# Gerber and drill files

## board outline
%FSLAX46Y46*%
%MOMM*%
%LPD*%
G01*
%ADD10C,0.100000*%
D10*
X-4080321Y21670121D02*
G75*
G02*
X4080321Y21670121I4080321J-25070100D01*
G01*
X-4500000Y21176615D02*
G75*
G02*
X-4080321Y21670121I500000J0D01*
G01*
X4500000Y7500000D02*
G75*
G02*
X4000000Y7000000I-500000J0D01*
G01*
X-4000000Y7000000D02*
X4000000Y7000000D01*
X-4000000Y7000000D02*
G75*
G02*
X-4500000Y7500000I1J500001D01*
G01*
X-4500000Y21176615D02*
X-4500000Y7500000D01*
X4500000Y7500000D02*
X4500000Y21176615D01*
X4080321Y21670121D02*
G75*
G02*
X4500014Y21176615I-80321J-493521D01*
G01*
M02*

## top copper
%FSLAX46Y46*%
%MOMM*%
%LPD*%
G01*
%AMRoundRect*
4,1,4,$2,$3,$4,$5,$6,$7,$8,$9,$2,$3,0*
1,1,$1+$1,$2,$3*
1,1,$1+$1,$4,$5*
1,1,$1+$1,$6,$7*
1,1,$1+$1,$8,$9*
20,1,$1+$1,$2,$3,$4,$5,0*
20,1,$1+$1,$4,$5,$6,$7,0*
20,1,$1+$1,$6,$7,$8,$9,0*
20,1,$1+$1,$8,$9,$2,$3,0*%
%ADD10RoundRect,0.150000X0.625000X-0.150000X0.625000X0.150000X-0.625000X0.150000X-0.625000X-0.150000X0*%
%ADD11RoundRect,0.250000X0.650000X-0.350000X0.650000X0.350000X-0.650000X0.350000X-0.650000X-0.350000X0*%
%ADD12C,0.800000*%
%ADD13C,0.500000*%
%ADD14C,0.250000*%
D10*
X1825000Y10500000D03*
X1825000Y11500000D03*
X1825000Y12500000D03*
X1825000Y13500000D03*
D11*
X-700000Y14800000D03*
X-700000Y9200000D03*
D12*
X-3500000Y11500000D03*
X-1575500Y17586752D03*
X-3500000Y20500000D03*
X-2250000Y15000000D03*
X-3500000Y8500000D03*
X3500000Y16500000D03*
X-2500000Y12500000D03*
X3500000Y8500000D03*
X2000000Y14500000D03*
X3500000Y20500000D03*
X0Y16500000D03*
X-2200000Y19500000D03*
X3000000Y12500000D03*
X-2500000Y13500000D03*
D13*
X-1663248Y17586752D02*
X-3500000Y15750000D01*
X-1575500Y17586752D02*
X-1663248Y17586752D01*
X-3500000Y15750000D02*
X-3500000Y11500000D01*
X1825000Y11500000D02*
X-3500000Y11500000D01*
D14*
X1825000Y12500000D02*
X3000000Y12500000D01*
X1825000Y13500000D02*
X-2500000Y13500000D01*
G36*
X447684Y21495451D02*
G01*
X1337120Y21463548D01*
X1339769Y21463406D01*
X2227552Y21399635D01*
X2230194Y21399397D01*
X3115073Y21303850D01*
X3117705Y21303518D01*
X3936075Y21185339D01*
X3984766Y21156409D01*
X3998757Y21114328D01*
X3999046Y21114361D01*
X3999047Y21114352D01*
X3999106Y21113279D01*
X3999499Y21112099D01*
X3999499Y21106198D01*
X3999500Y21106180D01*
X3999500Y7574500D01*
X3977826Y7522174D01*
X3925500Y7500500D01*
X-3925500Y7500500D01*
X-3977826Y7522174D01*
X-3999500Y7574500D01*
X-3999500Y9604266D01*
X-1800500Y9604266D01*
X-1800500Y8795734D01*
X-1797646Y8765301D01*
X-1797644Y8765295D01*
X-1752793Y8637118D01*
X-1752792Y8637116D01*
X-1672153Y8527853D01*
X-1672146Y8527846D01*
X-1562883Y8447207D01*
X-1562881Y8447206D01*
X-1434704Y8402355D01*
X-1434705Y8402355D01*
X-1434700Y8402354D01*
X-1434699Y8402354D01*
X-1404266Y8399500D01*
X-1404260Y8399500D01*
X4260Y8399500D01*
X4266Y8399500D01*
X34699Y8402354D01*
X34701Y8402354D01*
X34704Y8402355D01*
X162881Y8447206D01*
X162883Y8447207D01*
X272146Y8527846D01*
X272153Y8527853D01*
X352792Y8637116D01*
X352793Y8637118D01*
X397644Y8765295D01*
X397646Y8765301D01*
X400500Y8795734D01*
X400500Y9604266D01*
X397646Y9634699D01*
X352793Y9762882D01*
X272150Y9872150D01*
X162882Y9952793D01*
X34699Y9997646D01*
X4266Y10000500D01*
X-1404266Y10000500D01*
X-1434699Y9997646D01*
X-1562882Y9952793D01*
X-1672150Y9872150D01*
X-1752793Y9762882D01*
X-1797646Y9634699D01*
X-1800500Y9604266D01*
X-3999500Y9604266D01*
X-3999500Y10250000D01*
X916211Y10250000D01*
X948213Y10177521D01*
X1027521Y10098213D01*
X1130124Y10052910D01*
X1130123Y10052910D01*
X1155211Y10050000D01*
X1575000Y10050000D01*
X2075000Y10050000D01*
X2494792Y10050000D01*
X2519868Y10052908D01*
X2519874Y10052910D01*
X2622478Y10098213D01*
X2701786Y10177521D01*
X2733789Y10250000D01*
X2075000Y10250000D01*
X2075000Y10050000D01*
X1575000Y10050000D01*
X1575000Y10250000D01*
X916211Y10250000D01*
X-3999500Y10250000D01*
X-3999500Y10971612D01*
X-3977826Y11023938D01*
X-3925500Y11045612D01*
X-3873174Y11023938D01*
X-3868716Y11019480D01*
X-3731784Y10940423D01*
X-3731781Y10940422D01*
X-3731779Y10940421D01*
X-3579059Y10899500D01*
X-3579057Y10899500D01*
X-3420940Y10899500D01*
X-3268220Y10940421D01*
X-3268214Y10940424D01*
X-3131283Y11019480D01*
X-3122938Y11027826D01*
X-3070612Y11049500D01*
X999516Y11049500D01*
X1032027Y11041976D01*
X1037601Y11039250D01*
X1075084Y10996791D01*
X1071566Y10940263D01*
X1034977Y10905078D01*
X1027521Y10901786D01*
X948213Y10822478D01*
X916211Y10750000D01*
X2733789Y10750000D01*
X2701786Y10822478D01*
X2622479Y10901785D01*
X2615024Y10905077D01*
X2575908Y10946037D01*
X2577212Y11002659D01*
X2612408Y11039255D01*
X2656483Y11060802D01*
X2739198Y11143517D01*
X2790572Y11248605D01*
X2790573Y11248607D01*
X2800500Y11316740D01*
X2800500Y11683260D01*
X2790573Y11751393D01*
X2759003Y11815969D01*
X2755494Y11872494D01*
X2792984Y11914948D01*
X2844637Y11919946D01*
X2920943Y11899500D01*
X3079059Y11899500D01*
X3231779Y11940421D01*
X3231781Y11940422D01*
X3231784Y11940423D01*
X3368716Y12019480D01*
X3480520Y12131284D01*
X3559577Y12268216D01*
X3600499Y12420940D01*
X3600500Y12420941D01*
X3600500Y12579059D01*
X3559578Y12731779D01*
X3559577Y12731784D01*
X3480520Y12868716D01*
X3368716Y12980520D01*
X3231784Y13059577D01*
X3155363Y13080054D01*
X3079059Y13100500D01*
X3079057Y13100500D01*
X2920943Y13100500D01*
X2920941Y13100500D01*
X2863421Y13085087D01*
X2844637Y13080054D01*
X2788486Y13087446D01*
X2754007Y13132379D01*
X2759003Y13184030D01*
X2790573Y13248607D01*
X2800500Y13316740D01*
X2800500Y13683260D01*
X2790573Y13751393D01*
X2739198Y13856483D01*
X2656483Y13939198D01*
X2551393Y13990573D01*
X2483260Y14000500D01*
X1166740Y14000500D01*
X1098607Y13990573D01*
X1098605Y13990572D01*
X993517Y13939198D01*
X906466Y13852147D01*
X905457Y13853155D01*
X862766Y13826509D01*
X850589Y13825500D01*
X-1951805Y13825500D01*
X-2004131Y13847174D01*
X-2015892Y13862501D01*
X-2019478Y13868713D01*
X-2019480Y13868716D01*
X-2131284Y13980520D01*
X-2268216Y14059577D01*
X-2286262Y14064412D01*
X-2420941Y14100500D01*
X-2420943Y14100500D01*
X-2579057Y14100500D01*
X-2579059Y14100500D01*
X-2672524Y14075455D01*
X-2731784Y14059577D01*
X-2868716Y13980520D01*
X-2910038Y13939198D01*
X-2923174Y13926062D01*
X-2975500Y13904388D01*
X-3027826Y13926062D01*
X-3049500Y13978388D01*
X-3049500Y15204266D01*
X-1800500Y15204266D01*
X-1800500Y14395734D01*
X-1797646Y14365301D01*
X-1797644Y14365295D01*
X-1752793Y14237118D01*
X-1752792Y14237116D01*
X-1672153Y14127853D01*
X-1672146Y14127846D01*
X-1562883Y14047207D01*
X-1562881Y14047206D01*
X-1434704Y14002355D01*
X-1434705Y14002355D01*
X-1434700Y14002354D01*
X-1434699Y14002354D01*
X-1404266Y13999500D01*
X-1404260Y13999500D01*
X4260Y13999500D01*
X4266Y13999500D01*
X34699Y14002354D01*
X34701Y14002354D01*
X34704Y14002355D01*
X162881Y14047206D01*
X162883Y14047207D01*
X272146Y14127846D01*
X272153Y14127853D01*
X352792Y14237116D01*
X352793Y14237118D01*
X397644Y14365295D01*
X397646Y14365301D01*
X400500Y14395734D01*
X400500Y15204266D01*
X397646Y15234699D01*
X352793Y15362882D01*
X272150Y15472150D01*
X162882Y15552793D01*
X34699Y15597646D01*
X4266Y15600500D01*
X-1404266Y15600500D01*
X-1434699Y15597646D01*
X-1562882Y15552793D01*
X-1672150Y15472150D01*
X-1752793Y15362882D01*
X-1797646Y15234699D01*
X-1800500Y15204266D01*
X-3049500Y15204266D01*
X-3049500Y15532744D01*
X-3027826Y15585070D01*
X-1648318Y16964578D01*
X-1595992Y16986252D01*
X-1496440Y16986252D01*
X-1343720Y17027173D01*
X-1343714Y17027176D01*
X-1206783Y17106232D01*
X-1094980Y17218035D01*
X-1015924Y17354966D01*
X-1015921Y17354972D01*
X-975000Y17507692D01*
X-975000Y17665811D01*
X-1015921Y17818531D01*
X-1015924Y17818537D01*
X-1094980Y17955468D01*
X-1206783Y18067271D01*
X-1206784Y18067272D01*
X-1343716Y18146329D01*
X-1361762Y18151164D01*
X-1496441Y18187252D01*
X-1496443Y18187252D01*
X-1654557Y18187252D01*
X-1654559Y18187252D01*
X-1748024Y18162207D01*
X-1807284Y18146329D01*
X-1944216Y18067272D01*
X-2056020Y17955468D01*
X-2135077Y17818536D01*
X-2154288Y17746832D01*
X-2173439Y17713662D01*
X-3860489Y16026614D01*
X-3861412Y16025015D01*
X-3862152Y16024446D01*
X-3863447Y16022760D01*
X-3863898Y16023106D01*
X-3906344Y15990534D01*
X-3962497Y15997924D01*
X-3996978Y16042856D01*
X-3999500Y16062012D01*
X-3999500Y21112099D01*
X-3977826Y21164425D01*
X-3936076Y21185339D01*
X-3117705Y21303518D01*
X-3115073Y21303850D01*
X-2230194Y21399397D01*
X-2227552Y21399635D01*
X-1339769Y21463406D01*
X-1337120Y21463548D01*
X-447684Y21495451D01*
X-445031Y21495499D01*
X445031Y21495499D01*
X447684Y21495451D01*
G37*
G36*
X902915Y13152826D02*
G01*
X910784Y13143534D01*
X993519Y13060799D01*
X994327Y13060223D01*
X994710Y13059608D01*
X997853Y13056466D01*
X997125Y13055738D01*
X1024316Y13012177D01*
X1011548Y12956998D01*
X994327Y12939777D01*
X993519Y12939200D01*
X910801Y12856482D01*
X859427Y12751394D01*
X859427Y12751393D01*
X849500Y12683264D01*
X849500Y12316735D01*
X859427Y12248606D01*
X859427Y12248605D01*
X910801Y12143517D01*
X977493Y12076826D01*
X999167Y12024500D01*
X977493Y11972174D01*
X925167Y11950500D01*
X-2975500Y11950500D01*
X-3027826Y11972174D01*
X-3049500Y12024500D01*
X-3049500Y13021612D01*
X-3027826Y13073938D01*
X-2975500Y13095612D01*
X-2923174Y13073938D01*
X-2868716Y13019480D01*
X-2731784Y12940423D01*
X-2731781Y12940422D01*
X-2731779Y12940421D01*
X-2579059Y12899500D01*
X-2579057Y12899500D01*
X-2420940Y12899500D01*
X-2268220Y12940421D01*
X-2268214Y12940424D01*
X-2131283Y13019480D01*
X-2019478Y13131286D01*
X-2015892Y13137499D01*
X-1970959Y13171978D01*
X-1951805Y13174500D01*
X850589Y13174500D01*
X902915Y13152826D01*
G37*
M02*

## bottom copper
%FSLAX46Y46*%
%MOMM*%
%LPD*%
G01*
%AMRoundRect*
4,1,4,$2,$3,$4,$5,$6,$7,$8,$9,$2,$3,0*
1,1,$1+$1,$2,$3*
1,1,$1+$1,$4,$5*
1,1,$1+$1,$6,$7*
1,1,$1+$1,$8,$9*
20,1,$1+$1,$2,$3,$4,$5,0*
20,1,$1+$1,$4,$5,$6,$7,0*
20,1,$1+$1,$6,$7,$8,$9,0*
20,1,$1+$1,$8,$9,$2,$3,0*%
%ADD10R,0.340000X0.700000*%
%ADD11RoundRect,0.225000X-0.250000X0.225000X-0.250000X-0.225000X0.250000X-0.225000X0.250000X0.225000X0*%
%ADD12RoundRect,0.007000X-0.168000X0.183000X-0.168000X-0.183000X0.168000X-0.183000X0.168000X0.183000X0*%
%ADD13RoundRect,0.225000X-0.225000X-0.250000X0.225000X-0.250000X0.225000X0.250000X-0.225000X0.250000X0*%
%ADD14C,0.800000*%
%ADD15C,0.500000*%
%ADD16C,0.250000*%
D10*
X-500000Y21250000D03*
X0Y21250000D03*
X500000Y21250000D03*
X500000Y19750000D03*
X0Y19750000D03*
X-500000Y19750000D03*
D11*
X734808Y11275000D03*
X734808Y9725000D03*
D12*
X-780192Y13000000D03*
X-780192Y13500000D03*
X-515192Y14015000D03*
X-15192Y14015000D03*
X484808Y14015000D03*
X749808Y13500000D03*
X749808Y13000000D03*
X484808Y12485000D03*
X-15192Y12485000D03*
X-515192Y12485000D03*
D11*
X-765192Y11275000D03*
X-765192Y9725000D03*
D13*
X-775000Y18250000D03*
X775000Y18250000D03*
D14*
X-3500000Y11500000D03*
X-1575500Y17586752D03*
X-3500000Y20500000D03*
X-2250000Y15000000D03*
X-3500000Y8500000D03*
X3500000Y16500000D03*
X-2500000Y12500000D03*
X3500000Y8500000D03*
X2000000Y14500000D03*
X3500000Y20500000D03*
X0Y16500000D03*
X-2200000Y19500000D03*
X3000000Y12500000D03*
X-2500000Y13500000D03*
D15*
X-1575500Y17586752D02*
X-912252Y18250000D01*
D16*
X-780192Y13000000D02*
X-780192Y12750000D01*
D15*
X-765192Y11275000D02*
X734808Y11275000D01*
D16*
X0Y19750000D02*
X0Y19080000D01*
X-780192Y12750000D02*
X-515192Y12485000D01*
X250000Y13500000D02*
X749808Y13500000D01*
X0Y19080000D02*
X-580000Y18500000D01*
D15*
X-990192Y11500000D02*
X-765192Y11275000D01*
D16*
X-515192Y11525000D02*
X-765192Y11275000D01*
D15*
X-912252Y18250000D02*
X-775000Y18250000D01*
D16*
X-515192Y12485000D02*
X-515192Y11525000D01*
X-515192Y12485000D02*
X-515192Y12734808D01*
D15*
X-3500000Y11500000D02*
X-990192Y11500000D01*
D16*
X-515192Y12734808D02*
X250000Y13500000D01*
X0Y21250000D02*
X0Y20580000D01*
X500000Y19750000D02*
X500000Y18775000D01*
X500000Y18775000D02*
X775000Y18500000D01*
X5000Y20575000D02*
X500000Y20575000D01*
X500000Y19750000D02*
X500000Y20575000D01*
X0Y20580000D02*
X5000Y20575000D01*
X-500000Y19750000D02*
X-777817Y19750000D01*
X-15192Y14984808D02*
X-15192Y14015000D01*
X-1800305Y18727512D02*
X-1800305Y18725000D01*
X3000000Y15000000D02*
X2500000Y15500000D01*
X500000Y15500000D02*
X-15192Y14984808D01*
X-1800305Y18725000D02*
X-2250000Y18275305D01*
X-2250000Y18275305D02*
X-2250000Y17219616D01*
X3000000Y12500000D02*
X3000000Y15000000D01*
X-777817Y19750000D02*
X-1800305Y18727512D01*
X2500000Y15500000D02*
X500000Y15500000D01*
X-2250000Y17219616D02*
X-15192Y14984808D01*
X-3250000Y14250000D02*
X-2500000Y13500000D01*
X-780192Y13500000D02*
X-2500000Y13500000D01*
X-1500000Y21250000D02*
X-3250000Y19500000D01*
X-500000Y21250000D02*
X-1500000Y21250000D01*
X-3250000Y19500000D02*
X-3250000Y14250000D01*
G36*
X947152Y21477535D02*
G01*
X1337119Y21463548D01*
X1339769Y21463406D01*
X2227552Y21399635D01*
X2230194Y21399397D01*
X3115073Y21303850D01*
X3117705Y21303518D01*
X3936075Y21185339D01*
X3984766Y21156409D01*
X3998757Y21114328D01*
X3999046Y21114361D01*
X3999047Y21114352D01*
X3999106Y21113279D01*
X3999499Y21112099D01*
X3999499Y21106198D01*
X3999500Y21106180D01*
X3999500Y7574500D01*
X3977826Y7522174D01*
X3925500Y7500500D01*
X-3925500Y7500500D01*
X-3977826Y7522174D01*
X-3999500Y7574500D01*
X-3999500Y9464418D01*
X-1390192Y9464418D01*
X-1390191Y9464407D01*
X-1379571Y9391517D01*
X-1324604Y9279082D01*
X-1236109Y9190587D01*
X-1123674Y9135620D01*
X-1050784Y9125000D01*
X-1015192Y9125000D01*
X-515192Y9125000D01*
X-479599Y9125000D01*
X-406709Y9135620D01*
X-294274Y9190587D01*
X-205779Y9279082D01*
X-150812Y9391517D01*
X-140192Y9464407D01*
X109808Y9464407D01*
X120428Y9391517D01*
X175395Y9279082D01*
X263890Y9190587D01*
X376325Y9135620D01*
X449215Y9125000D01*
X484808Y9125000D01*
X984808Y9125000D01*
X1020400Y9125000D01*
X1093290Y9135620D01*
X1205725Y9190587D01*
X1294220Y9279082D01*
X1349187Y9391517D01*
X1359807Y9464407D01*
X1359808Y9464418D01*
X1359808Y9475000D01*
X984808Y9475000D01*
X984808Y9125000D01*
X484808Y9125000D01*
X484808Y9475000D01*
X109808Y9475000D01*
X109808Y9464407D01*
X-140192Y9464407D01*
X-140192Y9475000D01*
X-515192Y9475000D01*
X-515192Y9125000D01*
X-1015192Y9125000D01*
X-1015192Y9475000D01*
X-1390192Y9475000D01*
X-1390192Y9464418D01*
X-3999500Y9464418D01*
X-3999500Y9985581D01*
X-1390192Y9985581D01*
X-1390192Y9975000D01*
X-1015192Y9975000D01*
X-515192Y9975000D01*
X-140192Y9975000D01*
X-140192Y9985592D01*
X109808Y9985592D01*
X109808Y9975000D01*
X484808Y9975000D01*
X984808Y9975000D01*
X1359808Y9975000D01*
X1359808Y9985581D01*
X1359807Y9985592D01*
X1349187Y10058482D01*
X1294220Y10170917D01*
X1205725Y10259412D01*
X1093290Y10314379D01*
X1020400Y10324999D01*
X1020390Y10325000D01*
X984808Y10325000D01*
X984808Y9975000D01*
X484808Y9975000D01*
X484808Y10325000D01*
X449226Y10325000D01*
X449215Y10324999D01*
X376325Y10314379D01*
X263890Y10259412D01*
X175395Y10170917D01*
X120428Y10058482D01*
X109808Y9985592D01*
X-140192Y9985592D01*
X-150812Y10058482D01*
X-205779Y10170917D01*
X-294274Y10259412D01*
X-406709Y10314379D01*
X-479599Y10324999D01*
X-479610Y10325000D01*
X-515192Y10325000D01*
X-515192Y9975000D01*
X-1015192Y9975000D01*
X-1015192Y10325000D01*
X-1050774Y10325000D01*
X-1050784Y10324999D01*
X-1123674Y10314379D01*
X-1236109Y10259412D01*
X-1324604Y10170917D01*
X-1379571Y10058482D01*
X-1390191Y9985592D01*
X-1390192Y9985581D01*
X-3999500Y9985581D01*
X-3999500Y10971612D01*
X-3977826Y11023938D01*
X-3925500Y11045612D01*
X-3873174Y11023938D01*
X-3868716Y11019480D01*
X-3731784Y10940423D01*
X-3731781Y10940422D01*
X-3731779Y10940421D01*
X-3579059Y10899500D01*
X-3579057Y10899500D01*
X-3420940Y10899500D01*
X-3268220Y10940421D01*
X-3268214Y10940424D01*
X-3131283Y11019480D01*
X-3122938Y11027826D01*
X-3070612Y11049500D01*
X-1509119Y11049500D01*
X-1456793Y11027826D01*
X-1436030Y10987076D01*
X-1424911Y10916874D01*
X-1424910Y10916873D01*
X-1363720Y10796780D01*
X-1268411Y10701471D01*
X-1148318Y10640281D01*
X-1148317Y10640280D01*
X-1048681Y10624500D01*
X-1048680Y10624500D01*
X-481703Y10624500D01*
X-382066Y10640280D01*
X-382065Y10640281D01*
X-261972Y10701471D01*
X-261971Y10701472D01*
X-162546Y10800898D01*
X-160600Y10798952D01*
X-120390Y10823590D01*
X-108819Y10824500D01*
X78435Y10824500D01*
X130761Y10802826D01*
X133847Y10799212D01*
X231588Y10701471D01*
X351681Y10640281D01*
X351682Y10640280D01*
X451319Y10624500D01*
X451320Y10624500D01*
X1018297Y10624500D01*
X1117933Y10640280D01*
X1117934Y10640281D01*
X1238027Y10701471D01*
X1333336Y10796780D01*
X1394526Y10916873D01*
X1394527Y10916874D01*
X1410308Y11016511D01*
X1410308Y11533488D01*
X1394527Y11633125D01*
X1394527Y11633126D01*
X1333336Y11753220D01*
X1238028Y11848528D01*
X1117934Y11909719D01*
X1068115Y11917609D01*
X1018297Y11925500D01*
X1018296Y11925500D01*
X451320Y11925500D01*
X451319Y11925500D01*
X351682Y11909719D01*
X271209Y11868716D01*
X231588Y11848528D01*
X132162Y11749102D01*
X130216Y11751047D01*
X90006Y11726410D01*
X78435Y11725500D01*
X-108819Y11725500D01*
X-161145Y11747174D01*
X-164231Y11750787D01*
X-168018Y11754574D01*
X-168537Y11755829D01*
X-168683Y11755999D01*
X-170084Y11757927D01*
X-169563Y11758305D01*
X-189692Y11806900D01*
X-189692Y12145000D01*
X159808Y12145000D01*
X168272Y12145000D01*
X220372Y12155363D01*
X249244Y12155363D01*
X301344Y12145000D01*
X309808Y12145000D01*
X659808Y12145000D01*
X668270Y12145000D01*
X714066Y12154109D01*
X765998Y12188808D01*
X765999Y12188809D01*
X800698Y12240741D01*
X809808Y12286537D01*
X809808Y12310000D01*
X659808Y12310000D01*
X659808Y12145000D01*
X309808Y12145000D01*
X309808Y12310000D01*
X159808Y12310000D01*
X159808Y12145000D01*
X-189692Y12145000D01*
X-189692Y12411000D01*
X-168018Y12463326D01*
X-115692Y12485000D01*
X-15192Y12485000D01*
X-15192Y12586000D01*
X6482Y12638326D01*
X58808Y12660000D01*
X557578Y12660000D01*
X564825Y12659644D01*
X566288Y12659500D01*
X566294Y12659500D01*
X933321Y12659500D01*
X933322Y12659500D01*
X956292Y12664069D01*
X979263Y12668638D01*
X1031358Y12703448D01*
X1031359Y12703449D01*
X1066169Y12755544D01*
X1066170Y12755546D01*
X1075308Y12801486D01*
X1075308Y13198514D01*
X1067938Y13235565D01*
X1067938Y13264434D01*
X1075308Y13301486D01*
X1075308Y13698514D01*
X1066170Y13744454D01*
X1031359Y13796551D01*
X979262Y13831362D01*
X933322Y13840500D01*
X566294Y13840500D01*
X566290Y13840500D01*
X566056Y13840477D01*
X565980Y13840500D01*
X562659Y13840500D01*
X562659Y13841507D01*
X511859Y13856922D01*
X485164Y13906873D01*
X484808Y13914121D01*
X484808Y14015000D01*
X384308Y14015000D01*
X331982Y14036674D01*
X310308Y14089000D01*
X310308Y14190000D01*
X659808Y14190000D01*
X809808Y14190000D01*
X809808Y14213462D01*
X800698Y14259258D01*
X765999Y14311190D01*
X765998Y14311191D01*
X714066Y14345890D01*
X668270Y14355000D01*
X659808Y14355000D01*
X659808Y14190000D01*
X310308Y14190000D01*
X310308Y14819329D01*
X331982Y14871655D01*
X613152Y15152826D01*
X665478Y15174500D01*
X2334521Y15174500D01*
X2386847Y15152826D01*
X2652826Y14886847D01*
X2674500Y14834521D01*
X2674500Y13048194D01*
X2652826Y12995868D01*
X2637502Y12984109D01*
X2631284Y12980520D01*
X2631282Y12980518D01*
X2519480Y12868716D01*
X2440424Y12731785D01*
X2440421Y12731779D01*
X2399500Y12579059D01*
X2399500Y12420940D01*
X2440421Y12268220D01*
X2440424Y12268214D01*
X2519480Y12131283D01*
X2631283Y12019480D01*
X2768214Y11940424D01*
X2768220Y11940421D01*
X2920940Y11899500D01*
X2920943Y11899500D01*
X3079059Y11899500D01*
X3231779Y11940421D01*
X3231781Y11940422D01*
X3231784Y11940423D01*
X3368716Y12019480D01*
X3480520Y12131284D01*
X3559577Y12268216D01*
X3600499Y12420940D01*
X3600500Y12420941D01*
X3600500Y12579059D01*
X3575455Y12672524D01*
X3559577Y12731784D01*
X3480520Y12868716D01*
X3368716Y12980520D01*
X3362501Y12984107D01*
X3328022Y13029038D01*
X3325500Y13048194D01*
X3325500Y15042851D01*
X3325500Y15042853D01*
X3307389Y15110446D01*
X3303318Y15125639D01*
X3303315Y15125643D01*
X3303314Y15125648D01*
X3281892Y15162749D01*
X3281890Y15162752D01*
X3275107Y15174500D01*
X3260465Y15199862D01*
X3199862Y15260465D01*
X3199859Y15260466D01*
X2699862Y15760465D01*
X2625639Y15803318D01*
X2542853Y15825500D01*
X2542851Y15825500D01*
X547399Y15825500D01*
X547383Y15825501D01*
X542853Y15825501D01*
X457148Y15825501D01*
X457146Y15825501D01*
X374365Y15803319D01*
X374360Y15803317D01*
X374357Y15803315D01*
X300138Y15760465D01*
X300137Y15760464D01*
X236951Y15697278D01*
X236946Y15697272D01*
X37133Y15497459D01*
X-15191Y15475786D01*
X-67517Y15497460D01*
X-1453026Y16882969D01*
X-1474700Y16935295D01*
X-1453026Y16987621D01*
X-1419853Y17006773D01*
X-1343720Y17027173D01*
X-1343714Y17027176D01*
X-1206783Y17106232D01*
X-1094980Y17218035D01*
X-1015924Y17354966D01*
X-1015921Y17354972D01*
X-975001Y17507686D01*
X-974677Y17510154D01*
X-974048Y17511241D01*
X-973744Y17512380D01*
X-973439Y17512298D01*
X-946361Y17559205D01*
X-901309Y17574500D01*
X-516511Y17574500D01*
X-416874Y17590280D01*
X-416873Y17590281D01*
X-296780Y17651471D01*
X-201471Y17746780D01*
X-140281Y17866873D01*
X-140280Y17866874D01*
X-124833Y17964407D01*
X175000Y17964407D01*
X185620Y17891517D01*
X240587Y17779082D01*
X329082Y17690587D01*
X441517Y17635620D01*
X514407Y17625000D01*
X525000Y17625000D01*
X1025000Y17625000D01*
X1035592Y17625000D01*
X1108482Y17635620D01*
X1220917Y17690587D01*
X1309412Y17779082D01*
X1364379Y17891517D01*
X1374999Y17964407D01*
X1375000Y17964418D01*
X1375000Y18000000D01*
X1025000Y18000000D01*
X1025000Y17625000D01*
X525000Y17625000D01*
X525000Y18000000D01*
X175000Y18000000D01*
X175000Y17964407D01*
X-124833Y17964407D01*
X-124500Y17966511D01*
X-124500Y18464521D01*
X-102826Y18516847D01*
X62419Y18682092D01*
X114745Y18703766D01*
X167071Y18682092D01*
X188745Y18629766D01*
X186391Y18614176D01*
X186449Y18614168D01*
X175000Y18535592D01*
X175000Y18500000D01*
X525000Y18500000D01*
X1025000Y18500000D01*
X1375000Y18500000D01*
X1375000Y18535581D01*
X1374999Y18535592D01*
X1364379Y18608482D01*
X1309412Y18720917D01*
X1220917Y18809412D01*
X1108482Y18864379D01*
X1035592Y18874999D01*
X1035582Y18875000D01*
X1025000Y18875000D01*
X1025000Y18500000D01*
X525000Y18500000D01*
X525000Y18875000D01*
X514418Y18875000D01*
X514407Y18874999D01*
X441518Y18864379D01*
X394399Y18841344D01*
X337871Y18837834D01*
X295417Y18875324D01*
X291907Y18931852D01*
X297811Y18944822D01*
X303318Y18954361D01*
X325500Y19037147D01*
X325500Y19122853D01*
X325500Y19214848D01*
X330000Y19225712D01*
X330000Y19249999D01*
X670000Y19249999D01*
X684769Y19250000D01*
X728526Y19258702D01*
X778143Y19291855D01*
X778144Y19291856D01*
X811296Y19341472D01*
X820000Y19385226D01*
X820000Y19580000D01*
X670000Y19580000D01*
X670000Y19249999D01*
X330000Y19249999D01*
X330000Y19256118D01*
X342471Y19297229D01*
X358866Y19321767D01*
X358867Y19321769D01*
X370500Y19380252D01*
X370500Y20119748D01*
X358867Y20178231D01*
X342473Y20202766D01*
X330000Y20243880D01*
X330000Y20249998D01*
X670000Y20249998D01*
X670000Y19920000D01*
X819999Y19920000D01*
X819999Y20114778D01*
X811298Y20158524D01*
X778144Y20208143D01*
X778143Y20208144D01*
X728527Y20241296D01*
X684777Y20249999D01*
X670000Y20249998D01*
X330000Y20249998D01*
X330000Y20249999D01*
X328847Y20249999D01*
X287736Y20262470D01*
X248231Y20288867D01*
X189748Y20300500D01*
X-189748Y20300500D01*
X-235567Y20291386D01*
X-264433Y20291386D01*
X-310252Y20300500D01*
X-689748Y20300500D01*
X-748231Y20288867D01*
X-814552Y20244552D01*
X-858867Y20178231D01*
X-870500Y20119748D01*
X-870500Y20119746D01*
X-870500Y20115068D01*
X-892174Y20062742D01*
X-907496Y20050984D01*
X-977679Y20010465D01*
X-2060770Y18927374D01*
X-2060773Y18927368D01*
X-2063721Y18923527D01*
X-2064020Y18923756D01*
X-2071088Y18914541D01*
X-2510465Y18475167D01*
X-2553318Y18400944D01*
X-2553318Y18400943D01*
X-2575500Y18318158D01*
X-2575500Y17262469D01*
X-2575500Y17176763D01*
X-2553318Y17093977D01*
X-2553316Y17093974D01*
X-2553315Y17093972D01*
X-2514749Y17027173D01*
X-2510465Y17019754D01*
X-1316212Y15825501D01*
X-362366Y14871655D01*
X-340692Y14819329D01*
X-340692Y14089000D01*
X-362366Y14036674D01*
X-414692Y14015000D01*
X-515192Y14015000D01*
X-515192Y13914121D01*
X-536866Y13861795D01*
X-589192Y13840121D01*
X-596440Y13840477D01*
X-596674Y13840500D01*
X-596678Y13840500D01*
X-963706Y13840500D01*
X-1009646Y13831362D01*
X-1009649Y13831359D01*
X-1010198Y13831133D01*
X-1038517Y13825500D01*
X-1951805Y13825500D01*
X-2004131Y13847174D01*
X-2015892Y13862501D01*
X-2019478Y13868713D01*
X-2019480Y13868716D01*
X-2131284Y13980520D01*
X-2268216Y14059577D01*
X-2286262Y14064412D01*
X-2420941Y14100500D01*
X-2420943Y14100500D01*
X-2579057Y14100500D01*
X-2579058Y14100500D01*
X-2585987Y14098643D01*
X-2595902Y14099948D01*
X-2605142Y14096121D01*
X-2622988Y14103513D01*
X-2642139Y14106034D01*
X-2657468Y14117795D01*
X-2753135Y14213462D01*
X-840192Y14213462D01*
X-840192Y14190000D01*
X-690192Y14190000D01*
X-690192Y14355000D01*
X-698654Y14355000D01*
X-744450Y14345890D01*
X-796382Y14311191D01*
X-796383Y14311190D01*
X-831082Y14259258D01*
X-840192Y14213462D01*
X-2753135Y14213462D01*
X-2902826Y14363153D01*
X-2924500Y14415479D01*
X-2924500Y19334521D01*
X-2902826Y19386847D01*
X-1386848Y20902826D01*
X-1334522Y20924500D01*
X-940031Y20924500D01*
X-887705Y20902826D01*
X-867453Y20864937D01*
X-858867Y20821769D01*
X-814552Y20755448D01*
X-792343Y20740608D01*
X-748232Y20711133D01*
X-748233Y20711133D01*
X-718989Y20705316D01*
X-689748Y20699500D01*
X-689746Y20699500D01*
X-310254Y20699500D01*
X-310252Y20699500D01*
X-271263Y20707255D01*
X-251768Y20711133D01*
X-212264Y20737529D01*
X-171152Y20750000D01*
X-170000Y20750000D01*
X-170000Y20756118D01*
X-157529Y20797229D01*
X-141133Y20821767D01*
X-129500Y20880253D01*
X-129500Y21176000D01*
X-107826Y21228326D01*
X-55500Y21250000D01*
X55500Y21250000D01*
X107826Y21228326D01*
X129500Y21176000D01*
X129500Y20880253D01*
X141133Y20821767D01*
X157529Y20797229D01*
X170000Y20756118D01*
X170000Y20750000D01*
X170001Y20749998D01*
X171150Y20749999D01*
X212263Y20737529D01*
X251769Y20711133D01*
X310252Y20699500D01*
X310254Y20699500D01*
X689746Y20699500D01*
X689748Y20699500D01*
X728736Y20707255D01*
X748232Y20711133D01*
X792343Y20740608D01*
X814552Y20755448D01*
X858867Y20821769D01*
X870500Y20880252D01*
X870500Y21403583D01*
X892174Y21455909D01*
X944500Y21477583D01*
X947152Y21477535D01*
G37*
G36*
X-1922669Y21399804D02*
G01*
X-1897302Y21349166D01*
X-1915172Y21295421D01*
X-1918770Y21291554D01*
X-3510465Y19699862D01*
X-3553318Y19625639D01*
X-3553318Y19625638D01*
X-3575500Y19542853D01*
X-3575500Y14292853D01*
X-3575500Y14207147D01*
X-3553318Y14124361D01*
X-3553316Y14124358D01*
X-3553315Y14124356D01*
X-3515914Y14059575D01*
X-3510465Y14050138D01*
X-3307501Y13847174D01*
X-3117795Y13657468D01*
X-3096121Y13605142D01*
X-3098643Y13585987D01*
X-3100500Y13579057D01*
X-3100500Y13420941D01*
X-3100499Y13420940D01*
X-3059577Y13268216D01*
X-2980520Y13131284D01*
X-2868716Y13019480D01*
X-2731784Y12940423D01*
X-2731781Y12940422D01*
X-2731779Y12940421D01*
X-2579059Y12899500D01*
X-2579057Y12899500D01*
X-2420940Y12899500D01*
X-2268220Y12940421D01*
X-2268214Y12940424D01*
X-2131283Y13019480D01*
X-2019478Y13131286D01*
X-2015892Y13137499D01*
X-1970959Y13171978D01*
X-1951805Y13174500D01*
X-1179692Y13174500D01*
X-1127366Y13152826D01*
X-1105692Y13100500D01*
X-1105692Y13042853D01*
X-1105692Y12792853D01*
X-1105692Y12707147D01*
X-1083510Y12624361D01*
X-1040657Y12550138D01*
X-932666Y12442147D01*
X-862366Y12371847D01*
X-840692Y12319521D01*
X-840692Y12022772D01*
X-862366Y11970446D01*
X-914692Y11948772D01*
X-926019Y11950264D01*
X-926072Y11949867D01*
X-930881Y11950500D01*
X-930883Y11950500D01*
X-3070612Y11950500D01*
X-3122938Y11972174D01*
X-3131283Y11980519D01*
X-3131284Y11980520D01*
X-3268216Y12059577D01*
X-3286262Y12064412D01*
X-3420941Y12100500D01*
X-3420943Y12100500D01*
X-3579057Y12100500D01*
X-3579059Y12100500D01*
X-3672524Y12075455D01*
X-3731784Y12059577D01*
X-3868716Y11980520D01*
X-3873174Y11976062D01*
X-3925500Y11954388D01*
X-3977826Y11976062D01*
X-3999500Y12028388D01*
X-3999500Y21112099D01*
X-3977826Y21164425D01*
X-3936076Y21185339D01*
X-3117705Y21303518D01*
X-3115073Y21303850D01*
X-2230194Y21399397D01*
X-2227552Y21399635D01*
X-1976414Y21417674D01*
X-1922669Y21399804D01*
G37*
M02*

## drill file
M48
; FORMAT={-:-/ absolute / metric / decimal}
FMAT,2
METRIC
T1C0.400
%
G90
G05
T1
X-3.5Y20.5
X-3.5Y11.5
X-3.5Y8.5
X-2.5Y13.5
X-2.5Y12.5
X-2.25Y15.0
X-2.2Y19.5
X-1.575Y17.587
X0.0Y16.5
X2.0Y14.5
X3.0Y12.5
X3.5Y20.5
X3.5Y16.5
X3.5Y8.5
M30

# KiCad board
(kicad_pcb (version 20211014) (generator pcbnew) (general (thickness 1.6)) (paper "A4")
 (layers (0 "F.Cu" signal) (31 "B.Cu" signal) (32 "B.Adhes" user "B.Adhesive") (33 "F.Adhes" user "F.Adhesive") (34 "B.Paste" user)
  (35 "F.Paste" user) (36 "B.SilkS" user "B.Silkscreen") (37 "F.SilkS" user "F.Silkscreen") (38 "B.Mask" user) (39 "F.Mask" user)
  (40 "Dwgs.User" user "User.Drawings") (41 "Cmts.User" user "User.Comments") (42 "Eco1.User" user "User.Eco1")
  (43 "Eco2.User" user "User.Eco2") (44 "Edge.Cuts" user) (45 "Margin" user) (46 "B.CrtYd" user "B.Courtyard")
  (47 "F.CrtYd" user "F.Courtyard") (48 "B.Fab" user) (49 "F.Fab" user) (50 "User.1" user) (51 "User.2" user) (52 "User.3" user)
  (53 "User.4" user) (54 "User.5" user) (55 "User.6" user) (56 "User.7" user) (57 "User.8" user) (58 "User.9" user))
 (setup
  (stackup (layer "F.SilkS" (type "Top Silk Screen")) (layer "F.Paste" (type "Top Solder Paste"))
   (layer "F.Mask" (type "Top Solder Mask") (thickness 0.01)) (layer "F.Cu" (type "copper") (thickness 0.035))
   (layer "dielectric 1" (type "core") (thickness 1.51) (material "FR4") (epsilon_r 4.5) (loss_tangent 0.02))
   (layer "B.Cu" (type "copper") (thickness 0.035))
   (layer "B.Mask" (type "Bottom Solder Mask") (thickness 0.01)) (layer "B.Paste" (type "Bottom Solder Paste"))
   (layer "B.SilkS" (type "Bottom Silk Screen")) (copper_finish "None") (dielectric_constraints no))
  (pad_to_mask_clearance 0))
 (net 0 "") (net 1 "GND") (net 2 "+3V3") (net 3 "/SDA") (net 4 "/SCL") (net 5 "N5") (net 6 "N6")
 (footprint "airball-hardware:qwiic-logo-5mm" (layer "F.Cu") (at -3 -12 90)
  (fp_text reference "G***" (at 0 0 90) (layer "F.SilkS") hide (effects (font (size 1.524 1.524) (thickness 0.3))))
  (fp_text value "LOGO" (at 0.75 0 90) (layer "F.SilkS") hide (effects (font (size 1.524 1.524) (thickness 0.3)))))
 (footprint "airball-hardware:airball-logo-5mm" (layer "F.Cu") (at 0 -19)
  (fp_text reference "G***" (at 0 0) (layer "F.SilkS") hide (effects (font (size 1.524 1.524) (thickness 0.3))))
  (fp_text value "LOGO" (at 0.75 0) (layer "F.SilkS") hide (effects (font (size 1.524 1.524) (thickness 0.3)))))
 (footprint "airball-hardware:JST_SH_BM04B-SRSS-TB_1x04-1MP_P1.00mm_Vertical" (layer "F.Cu") (at 0.5 -12 90)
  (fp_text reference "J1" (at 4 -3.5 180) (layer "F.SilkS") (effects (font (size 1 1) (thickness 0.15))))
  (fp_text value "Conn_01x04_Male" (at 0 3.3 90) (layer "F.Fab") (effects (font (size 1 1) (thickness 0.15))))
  (pad "1" smd roundrect (at -1.5 1.325 90) (size 0.6 1.55) (layers "F.Cu" "F.Paste" "F.Mask") (roundrect_rratio 0.25) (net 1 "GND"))
  (pad "2" smd roundrect (at -0.5 1.325 90) (size 0.6 1.55) (layers "F.Cu" "F.Paste" "F.Mask") (roundrect_rratio 0.25) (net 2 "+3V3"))
  (pad "3" smd roundrect (at 0.5 1.325 90) (size 0.6 1.55) (layers "F.Cu" "F.Paste" "F.Mask") (roundrect_rratio 0.25) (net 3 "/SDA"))
  (pad "4" smd roundrect (at 1.5 1.325 90) (size 0.6 1.55) (layers "F.Cu" "F.Paste" "F.Mask") (roundrect_rratio 0.25) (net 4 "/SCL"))
  (pad "MP" smd roundrect (at 2.8 -1.2 90) (size 1.2 1.8) (layers "F.Cu" "F.Paste" "F.Mask") (roundrect_rratio 0.2083333333))
  (pad "MP" smd roundrect (at -2.8 -1.2 90) (size 1.2 1.8) (layers "F.Cu" "F.Paste" "F.Mask") (roundrect_rratio 0.2083333333)))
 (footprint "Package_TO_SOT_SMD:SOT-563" (layer "B.Cu") (at 0 -20.5 -90)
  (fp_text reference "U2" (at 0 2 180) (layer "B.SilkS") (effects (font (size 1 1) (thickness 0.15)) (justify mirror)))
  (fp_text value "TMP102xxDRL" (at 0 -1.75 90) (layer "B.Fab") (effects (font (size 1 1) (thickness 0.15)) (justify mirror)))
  (pad "1" smd rect (at -0.75 0.5 270) (size 0.7 0.34) (layers "B.Cu" "B.Paste" "B.Mask") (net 4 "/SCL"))
  (pad "2" smd rect (at -0.75 0 270) (size 0.7 0.34) (layers "B.Cu" "B.Paste" "B.Mask") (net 1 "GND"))
  (pad "3" smd rect (at -0.75 -0.5 270) (size 0.7 0.34) (layers "B.Cu" "B.Paste" "B.Mask") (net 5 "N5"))
  (pad "4" smd rect (at 0.75 -0.5 270) (size 0.7 0.34) (layers "B.Cu" "B.Paste" "B.Mask") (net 1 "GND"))
  (pad "5" smd rect (at 0.75 0 270) (size 0.7 0.34) (layers "B.Cu" "B.Paste" "B.Mask") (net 2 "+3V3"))
  (pad "6" smd rect (at 0.75 0.5 270) (size 0.7 0.34) (layers "B.Cu" "B.Paste" "B.Mask") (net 3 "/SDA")))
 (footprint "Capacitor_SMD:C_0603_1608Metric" (layer "B.Cu") (at 0.734808 -10.5 -90)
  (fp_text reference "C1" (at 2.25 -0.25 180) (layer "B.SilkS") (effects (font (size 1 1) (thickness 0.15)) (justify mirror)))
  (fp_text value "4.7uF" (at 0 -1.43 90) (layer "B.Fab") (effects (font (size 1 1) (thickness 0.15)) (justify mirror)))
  (pad "1" smd roundrect (at -0.775 0 270) (size 0.9 0.95) (layers "B.Cu" "B.Paste" "B.Mask") (roundrect_rratio 0.25) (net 2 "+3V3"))
  (pad "2" smd roundrect (at 0.775 0 270) (size 0.9 0.95) (layers "B.Cu" "B.Paste" "B.Mask") (roundrect_rratio 0.25) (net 1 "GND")))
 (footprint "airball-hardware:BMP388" (layer "B.Cu") (at -0.015192 -13.25) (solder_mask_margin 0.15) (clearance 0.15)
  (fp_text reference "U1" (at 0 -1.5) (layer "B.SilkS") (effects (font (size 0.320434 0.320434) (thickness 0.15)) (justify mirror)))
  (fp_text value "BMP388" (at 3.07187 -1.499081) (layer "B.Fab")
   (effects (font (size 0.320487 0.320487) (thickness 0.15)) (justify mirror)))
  (pad "1" smd roundrect (at -0.765 0.25 270) (size 0.38 0.35) (layers "B.Cu" "B.Paste" "B.Mask") (roundrect_rratio 0.02) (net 2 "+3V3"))
  (pad "2" smd roundrect (at -0.765 -0.25 270) (size 0.38 0.35) (layers "B.Cu" "B.Paste" "B.Mask") (roundrect_rratio 0.02) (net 4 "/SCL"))
  (pad "3" smd roundrect (at -0.5 -0.765 270) (size 0.38 0.35) (layers "B.Cu" "B.Paste" "B.Mask") (roundrect_rratio 0.02) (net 1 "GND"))
  (pad "4" smd roundrect (at 0 -0.765 270) (size 0.38 0.35) (layers "B.Cu" "B.Paste" "B.Mask") (roundrect_rratio 0.02) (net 3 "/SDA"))
  (pad "5" smd roundrect (at 0.5 -0.765 270) (size 0.38 0.35) (layers "B.Cu" "B.Paste" "B.Mask") (roundrect_rratio 0.02) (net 1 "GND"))
  (pad "6" smd roundrect (at 0.765 -0.25 270) (size 0.38 0.35) (layers "B.Cu" "B.Paste" "B.Mask") (roundrect_rratio 0.02) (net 2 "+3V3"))
  (pad "7" smd roundrect (at 0.765 0.25 270) (size 0.38 0.35) (layers "B.Cu" "B.Paste" "B.Mask") (roundrect_rratio 0.02) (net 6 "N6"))
  (pad "8" smd roundrect (at 0.5 0.765 270) (size 0.38 0.35) (layers "B.Cu" "B.Paste" "B.Mask") (roundrect_rratio 0.02) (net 1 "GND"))
  (pad "9" smd roundrect (at 0 0.765 270) (size 0.38 0.35) (layers "B.Cu" "B.Paste" "B.Mask") (roundrect_rratio 0.02) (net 1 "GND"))
  (pad "10" smd roundrect (at -0.5 0.765 270) (size 0.38 0.35) (layers "B.Cu" "B.Paste" "B.Mask") (roundrect_rratio 0.02) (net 2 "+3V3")))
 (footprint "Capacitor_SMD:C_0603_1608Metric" (layer "B.Cu") (at -0.765192 -10.5 -90)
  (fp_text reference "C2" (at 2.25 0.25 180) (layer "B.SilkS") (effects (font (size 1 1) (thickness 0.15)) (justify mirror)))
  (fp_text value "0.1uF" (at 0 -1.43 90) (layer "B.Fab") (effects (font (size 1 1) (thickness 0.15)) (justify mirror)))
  (pad "1" smd roundrect (at -0.775 0 270) (size 0.9 0.95) (layers "B.Cu" "B.Paste" "B.Mask") (roundrect_rratio 0.25) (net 2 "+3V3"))
  (pad "2" smd roundrect (at 0.775 0 270) (size 0.9 0.95) (layers "B.Cu" "B.Paste" "B.Mask") (roundrect_rratio 0.25) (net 1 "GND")))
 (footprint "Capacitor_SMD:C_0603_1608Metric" (layer "B.Cu") (at 0 -18.25)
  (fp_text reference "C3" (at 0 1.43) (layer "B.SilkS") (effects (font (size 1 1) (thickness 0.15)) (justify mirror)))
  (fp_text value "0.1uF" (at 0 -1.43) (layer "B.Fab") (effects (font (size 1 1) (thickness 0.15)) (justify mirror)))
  (pad "1" smd roundrect (at -0.775 0) (size 0.9 0.95) (layers "B.Cu" "B.Paste" "B.Mask") (roundrect_rratio 0.25) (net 2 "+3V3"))
  (pad "2" smd roundrect (at 0.775 0) (size 0.9 0.95) (layers "B.Cu" "B.Paste" "B.Mask") (roundrect_rratio 0.25) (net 1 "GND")))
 (gr_arc (start -4.080321 -21.670121) (mid 0 -22) (end 4.080321 -21.670121) (layer "Edge.Cuts") (width 0.1))
 (gr_arc (start -4.5 -21.176615) (mid -4.380894 -21.500528) (end -4.080321 -21.670121) (layer "Edge.Cuts") (width 0.1))
 (gr_arc (start 4.5 -7.5) (mid 4.353553 -7.146447) (end 4 -7) (layer "Edge.Cuts") (width 0.1))
 (gr_line (start -4 -7) (end 4 -7) (layer "Edge.Cuts") (width 0.1))
 (gr_arc (start -4 -7) (mid -4.353553 -7.146447) (end -4.5 -7.5) (layer "Edge.Cuts") (width 0.1))
 (gr_line (start -4.5 -21.176615) (end -4.5 -7.5) (layer "Edge.Cuts") (width 0.1))
 (gr_line (start 4.5 -7.5) (end 4.5 -21.176615) (layer "Edge.Cuts") (width 0.1))
 (gr_arc (start 4.080321 -21.670121) (mid 4.380896 -21.500528) (end 4.5 -21.176615) (layer "Edge.Cuts") (width 0.1))
 (segment (start -1.663248 -17.586752) (end -3.5 -15.75) (width 0.5) (layer "F.Cu") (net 2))
 (segment (start -1.5755 -17.586752) (end -1.663248 -17.586752) (width 0.5) (layer "F.Cu") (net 2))
 (segment (start -3.5 -15.75) (end -3.5 -11.5) (width 0.5) (layer "F.Cu") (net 2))
 (segment (start 1.825 -11.5) (end -3.5 -11.5) (width 0.5) (layer "F.Cu") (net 2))
 (via (at -3.5 -11.5) (size 0.8) (drill 0.4) (layers "F.Cu" "B.Cu") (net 2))
 (via (at -1.5755 -17.586752) (size 0.8) (drill 0.4) (layers "F.Cu" "B.Cu") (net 2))
 (segment (start -1.5755 -17.586752) (end -0.912252 -18.25) (width 0.5) (layer "B.Cu") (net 2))
 (segment (start -0.780192 -13) (end -0.780192 -12.75) (width 0.25) (layer "B.Cu") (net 2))
 (segment (start -0.765192 -11.275) (end 0.734808 -11.275) (width 0.5) (layer "B.Cu") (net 2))
 (segment (start 0 -19.75) (end 0 -19.08) (width 0.25) (layer "B.Cu") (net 2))
 (segment (start -0.780192 -12.75) (end -0.515192 -12.485) (width 0.25) (layer "B.Cu") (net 2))
 (segment (start 0.25 -13.5) (end 0.749808 -13.5) (width 0.25) (layer "B.Cu") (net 2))
 (segment (start 0 -19.08) (end -0.58 -18.5) (width 0.25) (layer "B.Cu") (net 2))
 (segment (start -0.990192 -11.5) (end -0.765192 -11.275) (width 0.5) (layer "B.Cu") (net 2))
 (segment (start -0.515192 -11.525) (end -0.765192 -11.275) (width 0.25) (layer "B.Cu") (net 2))
 (segment (start -0.912252 -18.25) (end -0.775 -18.25) (width 0.5) (layer "B.Cu") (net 2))
 (segment (start -0.515192 -12.485) (end -0.515192 -11.525) (width 0.25) (layer "B.Cu") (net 2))
 (segment (start -0.515192 -12.485) (end -0.515192 -12.734808) (width 0.25) (layer "B.Cu") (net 2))
 (segment (start -3.5 -11.5) (end -0.990192 -11.5) (width 0.5) (layer "B.Cu") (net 2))
 (segment (start -0.515192 -12.734808) (end 0.25 -13.5) (width 0.25) (layer "B.Cu") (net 2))
 (via (at -3.5 -20.5) (size 0.8) (drill 0.4) (layers "F.Cu" "B.Cu") (free) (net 1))
 (via (at -2.25 -15) (size 0.8) (drill 0.4) (layers "F.Cu" "B.Cu") (free) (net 1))
 (via (at -3.5 -8.5) (size 0.8) (drill 0.4) (layers "F.Cu" "B.Cu") (free) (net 1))
 (via (at 3.5 -16.5) (size 0.8) (drill 0.4) (layers "F.Cu" "B.Cu") (free) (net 1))
 (via (at -2.5 -12.5) (size 0.8) (drill 0.4) (layers "F.Cu" "B.Cu") (free) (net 1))
 (via (at 3.5 -8.5) (size 0.8) (drill 0.4) (layers "F.Cu" "B.Cu") (free) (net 1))
 (via (at 2 -14.5) (size 0.8) (drill 0.4) (layers "F.Cu" "B.Cu") (free) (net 1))
 (via (at 3.5 -20.5) (size 0.8) (drill 0.4) (layers "F.Cu" "B.Cu") (free) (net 1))
 (via (at 0 -16.5) (size 0.8) (drill 0.4) (layers "F.Cu" "B.Cu") (free) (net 1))
 (via (at -2.2 -19.5) (size 0.8) (drill 0.4) (layers "F.Cu" "B.Cu") (free) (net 1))
 (segment (start 0 -21.25) (end 0 -20.58) (width 0.25) (layer "B.Cu") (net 1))
 (segment (start 0.5 -19.75) (end 0.5 -18.775) (width 0.25) (layer "B.Cu") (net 1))
 (segment (start 0.5 -18.775) (end 0.775 -18.5) (width 0.25) (layer "B.Cu") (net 1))
 (segment (start 0.005 -20.575) (end 0.5 -20.575) (width 0.25) (layer "B.Cu") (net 1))
 (segment (start 0.5 -19.75) (end 0.5 -20.575) (width 0.25) (layer "B.Cu") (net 1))
 (segment (start 0 -20.58) (end 0.005 -20.575) (width 0.25) (layer "B.Cu") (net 1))
 (segment (start 1.825 -12.5) (end 3 -12.5) (width 0.25) (layer "F.Cu") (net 3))
 (via (at 3 -12.5) (size 0.8) (drill 0.4) (layers "F.Cu" "B.Cu") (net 3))
 (segment (start -0.5 -19.75) (end -0.777817 -19.75) (width 0.25) (layer "B.Cu") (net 3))
 (segment (start -0.015192 -14.984808) (end -0.015192 -14.015) (width 0.25) (layer "B.Cu") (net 3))
 (segment (start -1.800305 -18.727512) (end -1.800305 -18.725) (width 0.25) (layer "B.Cu") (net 3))
 (segment (start 3 -15) (end 2.5 -15.5) (width 0.25) (layer "B.Cu") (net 3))
 (segment (start 0.5 -15.5) (end -0.015192 -14.984808) (width 0.25) (layer "B.Cu") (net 3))
 (segment (start -1.800305 -18.725) (end -2.25 -18.275305) (width 0.25) (layer "B.Cu") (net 3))
 (segment (start -2.25 -18.275305) (end -2.25 -17.219616) (width 0.25) (layer "B.Cu") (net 3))
 (segment (start 3 -12.5) (end 3 -15) (width 0.25) (layer "B.Cu") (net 3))
 (segment (start -0.777817 -19.75) (end -1.800305 -18.727512) (width 0.25) (layer "B.Cu") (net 3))
 (segment (start 2.5 -15.5) (end 0.5 -15.5) (width 0.25) (layer "B.Cu") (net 3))
 (segment (start -2.25 -17.219616) (end -0.015192 -14.984808) (width 0.25) (layer "B.Cu") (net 3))
 (segment (start 1.825 -13.5) (end -2.5 -13.5) (width 0.25) (layer "F.Cu") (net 4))
 (via (at -2.5 -13.5) (size 0.8) (drill 0.4) (layers "F.Cu" "B.Cu") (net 4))
 (segment (start -3.25 -14.25) (end -2.5 -13.5) (width 0.25) (layer "B.Cu") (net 4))
 (segment (start -0.780192 -13.5) (end -2.5 -13.5) (width 0.25) (layer "B.Cu") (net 4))
 (segment (start -1.5 -21.25) (end -3.25 -19.5) (width 0.25) (layer "B.Cu") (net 4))
 (segment (start -0.5 -21.25) (end -1.5 -21.25) (width 0.25) (layer "B.Cu") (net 4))
 (segment (start -3.25 -19.5) (end -3.25 -14.25) (width 0.25) (layer "B.Cu") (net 4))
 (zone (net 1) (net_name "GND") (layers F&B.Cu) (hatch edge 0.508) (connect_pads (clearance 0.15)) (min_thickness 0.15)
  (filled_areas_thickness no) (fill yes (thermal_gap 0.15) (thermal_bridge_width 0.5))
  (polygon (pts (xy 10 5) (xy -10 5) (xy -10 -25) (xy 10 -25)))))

